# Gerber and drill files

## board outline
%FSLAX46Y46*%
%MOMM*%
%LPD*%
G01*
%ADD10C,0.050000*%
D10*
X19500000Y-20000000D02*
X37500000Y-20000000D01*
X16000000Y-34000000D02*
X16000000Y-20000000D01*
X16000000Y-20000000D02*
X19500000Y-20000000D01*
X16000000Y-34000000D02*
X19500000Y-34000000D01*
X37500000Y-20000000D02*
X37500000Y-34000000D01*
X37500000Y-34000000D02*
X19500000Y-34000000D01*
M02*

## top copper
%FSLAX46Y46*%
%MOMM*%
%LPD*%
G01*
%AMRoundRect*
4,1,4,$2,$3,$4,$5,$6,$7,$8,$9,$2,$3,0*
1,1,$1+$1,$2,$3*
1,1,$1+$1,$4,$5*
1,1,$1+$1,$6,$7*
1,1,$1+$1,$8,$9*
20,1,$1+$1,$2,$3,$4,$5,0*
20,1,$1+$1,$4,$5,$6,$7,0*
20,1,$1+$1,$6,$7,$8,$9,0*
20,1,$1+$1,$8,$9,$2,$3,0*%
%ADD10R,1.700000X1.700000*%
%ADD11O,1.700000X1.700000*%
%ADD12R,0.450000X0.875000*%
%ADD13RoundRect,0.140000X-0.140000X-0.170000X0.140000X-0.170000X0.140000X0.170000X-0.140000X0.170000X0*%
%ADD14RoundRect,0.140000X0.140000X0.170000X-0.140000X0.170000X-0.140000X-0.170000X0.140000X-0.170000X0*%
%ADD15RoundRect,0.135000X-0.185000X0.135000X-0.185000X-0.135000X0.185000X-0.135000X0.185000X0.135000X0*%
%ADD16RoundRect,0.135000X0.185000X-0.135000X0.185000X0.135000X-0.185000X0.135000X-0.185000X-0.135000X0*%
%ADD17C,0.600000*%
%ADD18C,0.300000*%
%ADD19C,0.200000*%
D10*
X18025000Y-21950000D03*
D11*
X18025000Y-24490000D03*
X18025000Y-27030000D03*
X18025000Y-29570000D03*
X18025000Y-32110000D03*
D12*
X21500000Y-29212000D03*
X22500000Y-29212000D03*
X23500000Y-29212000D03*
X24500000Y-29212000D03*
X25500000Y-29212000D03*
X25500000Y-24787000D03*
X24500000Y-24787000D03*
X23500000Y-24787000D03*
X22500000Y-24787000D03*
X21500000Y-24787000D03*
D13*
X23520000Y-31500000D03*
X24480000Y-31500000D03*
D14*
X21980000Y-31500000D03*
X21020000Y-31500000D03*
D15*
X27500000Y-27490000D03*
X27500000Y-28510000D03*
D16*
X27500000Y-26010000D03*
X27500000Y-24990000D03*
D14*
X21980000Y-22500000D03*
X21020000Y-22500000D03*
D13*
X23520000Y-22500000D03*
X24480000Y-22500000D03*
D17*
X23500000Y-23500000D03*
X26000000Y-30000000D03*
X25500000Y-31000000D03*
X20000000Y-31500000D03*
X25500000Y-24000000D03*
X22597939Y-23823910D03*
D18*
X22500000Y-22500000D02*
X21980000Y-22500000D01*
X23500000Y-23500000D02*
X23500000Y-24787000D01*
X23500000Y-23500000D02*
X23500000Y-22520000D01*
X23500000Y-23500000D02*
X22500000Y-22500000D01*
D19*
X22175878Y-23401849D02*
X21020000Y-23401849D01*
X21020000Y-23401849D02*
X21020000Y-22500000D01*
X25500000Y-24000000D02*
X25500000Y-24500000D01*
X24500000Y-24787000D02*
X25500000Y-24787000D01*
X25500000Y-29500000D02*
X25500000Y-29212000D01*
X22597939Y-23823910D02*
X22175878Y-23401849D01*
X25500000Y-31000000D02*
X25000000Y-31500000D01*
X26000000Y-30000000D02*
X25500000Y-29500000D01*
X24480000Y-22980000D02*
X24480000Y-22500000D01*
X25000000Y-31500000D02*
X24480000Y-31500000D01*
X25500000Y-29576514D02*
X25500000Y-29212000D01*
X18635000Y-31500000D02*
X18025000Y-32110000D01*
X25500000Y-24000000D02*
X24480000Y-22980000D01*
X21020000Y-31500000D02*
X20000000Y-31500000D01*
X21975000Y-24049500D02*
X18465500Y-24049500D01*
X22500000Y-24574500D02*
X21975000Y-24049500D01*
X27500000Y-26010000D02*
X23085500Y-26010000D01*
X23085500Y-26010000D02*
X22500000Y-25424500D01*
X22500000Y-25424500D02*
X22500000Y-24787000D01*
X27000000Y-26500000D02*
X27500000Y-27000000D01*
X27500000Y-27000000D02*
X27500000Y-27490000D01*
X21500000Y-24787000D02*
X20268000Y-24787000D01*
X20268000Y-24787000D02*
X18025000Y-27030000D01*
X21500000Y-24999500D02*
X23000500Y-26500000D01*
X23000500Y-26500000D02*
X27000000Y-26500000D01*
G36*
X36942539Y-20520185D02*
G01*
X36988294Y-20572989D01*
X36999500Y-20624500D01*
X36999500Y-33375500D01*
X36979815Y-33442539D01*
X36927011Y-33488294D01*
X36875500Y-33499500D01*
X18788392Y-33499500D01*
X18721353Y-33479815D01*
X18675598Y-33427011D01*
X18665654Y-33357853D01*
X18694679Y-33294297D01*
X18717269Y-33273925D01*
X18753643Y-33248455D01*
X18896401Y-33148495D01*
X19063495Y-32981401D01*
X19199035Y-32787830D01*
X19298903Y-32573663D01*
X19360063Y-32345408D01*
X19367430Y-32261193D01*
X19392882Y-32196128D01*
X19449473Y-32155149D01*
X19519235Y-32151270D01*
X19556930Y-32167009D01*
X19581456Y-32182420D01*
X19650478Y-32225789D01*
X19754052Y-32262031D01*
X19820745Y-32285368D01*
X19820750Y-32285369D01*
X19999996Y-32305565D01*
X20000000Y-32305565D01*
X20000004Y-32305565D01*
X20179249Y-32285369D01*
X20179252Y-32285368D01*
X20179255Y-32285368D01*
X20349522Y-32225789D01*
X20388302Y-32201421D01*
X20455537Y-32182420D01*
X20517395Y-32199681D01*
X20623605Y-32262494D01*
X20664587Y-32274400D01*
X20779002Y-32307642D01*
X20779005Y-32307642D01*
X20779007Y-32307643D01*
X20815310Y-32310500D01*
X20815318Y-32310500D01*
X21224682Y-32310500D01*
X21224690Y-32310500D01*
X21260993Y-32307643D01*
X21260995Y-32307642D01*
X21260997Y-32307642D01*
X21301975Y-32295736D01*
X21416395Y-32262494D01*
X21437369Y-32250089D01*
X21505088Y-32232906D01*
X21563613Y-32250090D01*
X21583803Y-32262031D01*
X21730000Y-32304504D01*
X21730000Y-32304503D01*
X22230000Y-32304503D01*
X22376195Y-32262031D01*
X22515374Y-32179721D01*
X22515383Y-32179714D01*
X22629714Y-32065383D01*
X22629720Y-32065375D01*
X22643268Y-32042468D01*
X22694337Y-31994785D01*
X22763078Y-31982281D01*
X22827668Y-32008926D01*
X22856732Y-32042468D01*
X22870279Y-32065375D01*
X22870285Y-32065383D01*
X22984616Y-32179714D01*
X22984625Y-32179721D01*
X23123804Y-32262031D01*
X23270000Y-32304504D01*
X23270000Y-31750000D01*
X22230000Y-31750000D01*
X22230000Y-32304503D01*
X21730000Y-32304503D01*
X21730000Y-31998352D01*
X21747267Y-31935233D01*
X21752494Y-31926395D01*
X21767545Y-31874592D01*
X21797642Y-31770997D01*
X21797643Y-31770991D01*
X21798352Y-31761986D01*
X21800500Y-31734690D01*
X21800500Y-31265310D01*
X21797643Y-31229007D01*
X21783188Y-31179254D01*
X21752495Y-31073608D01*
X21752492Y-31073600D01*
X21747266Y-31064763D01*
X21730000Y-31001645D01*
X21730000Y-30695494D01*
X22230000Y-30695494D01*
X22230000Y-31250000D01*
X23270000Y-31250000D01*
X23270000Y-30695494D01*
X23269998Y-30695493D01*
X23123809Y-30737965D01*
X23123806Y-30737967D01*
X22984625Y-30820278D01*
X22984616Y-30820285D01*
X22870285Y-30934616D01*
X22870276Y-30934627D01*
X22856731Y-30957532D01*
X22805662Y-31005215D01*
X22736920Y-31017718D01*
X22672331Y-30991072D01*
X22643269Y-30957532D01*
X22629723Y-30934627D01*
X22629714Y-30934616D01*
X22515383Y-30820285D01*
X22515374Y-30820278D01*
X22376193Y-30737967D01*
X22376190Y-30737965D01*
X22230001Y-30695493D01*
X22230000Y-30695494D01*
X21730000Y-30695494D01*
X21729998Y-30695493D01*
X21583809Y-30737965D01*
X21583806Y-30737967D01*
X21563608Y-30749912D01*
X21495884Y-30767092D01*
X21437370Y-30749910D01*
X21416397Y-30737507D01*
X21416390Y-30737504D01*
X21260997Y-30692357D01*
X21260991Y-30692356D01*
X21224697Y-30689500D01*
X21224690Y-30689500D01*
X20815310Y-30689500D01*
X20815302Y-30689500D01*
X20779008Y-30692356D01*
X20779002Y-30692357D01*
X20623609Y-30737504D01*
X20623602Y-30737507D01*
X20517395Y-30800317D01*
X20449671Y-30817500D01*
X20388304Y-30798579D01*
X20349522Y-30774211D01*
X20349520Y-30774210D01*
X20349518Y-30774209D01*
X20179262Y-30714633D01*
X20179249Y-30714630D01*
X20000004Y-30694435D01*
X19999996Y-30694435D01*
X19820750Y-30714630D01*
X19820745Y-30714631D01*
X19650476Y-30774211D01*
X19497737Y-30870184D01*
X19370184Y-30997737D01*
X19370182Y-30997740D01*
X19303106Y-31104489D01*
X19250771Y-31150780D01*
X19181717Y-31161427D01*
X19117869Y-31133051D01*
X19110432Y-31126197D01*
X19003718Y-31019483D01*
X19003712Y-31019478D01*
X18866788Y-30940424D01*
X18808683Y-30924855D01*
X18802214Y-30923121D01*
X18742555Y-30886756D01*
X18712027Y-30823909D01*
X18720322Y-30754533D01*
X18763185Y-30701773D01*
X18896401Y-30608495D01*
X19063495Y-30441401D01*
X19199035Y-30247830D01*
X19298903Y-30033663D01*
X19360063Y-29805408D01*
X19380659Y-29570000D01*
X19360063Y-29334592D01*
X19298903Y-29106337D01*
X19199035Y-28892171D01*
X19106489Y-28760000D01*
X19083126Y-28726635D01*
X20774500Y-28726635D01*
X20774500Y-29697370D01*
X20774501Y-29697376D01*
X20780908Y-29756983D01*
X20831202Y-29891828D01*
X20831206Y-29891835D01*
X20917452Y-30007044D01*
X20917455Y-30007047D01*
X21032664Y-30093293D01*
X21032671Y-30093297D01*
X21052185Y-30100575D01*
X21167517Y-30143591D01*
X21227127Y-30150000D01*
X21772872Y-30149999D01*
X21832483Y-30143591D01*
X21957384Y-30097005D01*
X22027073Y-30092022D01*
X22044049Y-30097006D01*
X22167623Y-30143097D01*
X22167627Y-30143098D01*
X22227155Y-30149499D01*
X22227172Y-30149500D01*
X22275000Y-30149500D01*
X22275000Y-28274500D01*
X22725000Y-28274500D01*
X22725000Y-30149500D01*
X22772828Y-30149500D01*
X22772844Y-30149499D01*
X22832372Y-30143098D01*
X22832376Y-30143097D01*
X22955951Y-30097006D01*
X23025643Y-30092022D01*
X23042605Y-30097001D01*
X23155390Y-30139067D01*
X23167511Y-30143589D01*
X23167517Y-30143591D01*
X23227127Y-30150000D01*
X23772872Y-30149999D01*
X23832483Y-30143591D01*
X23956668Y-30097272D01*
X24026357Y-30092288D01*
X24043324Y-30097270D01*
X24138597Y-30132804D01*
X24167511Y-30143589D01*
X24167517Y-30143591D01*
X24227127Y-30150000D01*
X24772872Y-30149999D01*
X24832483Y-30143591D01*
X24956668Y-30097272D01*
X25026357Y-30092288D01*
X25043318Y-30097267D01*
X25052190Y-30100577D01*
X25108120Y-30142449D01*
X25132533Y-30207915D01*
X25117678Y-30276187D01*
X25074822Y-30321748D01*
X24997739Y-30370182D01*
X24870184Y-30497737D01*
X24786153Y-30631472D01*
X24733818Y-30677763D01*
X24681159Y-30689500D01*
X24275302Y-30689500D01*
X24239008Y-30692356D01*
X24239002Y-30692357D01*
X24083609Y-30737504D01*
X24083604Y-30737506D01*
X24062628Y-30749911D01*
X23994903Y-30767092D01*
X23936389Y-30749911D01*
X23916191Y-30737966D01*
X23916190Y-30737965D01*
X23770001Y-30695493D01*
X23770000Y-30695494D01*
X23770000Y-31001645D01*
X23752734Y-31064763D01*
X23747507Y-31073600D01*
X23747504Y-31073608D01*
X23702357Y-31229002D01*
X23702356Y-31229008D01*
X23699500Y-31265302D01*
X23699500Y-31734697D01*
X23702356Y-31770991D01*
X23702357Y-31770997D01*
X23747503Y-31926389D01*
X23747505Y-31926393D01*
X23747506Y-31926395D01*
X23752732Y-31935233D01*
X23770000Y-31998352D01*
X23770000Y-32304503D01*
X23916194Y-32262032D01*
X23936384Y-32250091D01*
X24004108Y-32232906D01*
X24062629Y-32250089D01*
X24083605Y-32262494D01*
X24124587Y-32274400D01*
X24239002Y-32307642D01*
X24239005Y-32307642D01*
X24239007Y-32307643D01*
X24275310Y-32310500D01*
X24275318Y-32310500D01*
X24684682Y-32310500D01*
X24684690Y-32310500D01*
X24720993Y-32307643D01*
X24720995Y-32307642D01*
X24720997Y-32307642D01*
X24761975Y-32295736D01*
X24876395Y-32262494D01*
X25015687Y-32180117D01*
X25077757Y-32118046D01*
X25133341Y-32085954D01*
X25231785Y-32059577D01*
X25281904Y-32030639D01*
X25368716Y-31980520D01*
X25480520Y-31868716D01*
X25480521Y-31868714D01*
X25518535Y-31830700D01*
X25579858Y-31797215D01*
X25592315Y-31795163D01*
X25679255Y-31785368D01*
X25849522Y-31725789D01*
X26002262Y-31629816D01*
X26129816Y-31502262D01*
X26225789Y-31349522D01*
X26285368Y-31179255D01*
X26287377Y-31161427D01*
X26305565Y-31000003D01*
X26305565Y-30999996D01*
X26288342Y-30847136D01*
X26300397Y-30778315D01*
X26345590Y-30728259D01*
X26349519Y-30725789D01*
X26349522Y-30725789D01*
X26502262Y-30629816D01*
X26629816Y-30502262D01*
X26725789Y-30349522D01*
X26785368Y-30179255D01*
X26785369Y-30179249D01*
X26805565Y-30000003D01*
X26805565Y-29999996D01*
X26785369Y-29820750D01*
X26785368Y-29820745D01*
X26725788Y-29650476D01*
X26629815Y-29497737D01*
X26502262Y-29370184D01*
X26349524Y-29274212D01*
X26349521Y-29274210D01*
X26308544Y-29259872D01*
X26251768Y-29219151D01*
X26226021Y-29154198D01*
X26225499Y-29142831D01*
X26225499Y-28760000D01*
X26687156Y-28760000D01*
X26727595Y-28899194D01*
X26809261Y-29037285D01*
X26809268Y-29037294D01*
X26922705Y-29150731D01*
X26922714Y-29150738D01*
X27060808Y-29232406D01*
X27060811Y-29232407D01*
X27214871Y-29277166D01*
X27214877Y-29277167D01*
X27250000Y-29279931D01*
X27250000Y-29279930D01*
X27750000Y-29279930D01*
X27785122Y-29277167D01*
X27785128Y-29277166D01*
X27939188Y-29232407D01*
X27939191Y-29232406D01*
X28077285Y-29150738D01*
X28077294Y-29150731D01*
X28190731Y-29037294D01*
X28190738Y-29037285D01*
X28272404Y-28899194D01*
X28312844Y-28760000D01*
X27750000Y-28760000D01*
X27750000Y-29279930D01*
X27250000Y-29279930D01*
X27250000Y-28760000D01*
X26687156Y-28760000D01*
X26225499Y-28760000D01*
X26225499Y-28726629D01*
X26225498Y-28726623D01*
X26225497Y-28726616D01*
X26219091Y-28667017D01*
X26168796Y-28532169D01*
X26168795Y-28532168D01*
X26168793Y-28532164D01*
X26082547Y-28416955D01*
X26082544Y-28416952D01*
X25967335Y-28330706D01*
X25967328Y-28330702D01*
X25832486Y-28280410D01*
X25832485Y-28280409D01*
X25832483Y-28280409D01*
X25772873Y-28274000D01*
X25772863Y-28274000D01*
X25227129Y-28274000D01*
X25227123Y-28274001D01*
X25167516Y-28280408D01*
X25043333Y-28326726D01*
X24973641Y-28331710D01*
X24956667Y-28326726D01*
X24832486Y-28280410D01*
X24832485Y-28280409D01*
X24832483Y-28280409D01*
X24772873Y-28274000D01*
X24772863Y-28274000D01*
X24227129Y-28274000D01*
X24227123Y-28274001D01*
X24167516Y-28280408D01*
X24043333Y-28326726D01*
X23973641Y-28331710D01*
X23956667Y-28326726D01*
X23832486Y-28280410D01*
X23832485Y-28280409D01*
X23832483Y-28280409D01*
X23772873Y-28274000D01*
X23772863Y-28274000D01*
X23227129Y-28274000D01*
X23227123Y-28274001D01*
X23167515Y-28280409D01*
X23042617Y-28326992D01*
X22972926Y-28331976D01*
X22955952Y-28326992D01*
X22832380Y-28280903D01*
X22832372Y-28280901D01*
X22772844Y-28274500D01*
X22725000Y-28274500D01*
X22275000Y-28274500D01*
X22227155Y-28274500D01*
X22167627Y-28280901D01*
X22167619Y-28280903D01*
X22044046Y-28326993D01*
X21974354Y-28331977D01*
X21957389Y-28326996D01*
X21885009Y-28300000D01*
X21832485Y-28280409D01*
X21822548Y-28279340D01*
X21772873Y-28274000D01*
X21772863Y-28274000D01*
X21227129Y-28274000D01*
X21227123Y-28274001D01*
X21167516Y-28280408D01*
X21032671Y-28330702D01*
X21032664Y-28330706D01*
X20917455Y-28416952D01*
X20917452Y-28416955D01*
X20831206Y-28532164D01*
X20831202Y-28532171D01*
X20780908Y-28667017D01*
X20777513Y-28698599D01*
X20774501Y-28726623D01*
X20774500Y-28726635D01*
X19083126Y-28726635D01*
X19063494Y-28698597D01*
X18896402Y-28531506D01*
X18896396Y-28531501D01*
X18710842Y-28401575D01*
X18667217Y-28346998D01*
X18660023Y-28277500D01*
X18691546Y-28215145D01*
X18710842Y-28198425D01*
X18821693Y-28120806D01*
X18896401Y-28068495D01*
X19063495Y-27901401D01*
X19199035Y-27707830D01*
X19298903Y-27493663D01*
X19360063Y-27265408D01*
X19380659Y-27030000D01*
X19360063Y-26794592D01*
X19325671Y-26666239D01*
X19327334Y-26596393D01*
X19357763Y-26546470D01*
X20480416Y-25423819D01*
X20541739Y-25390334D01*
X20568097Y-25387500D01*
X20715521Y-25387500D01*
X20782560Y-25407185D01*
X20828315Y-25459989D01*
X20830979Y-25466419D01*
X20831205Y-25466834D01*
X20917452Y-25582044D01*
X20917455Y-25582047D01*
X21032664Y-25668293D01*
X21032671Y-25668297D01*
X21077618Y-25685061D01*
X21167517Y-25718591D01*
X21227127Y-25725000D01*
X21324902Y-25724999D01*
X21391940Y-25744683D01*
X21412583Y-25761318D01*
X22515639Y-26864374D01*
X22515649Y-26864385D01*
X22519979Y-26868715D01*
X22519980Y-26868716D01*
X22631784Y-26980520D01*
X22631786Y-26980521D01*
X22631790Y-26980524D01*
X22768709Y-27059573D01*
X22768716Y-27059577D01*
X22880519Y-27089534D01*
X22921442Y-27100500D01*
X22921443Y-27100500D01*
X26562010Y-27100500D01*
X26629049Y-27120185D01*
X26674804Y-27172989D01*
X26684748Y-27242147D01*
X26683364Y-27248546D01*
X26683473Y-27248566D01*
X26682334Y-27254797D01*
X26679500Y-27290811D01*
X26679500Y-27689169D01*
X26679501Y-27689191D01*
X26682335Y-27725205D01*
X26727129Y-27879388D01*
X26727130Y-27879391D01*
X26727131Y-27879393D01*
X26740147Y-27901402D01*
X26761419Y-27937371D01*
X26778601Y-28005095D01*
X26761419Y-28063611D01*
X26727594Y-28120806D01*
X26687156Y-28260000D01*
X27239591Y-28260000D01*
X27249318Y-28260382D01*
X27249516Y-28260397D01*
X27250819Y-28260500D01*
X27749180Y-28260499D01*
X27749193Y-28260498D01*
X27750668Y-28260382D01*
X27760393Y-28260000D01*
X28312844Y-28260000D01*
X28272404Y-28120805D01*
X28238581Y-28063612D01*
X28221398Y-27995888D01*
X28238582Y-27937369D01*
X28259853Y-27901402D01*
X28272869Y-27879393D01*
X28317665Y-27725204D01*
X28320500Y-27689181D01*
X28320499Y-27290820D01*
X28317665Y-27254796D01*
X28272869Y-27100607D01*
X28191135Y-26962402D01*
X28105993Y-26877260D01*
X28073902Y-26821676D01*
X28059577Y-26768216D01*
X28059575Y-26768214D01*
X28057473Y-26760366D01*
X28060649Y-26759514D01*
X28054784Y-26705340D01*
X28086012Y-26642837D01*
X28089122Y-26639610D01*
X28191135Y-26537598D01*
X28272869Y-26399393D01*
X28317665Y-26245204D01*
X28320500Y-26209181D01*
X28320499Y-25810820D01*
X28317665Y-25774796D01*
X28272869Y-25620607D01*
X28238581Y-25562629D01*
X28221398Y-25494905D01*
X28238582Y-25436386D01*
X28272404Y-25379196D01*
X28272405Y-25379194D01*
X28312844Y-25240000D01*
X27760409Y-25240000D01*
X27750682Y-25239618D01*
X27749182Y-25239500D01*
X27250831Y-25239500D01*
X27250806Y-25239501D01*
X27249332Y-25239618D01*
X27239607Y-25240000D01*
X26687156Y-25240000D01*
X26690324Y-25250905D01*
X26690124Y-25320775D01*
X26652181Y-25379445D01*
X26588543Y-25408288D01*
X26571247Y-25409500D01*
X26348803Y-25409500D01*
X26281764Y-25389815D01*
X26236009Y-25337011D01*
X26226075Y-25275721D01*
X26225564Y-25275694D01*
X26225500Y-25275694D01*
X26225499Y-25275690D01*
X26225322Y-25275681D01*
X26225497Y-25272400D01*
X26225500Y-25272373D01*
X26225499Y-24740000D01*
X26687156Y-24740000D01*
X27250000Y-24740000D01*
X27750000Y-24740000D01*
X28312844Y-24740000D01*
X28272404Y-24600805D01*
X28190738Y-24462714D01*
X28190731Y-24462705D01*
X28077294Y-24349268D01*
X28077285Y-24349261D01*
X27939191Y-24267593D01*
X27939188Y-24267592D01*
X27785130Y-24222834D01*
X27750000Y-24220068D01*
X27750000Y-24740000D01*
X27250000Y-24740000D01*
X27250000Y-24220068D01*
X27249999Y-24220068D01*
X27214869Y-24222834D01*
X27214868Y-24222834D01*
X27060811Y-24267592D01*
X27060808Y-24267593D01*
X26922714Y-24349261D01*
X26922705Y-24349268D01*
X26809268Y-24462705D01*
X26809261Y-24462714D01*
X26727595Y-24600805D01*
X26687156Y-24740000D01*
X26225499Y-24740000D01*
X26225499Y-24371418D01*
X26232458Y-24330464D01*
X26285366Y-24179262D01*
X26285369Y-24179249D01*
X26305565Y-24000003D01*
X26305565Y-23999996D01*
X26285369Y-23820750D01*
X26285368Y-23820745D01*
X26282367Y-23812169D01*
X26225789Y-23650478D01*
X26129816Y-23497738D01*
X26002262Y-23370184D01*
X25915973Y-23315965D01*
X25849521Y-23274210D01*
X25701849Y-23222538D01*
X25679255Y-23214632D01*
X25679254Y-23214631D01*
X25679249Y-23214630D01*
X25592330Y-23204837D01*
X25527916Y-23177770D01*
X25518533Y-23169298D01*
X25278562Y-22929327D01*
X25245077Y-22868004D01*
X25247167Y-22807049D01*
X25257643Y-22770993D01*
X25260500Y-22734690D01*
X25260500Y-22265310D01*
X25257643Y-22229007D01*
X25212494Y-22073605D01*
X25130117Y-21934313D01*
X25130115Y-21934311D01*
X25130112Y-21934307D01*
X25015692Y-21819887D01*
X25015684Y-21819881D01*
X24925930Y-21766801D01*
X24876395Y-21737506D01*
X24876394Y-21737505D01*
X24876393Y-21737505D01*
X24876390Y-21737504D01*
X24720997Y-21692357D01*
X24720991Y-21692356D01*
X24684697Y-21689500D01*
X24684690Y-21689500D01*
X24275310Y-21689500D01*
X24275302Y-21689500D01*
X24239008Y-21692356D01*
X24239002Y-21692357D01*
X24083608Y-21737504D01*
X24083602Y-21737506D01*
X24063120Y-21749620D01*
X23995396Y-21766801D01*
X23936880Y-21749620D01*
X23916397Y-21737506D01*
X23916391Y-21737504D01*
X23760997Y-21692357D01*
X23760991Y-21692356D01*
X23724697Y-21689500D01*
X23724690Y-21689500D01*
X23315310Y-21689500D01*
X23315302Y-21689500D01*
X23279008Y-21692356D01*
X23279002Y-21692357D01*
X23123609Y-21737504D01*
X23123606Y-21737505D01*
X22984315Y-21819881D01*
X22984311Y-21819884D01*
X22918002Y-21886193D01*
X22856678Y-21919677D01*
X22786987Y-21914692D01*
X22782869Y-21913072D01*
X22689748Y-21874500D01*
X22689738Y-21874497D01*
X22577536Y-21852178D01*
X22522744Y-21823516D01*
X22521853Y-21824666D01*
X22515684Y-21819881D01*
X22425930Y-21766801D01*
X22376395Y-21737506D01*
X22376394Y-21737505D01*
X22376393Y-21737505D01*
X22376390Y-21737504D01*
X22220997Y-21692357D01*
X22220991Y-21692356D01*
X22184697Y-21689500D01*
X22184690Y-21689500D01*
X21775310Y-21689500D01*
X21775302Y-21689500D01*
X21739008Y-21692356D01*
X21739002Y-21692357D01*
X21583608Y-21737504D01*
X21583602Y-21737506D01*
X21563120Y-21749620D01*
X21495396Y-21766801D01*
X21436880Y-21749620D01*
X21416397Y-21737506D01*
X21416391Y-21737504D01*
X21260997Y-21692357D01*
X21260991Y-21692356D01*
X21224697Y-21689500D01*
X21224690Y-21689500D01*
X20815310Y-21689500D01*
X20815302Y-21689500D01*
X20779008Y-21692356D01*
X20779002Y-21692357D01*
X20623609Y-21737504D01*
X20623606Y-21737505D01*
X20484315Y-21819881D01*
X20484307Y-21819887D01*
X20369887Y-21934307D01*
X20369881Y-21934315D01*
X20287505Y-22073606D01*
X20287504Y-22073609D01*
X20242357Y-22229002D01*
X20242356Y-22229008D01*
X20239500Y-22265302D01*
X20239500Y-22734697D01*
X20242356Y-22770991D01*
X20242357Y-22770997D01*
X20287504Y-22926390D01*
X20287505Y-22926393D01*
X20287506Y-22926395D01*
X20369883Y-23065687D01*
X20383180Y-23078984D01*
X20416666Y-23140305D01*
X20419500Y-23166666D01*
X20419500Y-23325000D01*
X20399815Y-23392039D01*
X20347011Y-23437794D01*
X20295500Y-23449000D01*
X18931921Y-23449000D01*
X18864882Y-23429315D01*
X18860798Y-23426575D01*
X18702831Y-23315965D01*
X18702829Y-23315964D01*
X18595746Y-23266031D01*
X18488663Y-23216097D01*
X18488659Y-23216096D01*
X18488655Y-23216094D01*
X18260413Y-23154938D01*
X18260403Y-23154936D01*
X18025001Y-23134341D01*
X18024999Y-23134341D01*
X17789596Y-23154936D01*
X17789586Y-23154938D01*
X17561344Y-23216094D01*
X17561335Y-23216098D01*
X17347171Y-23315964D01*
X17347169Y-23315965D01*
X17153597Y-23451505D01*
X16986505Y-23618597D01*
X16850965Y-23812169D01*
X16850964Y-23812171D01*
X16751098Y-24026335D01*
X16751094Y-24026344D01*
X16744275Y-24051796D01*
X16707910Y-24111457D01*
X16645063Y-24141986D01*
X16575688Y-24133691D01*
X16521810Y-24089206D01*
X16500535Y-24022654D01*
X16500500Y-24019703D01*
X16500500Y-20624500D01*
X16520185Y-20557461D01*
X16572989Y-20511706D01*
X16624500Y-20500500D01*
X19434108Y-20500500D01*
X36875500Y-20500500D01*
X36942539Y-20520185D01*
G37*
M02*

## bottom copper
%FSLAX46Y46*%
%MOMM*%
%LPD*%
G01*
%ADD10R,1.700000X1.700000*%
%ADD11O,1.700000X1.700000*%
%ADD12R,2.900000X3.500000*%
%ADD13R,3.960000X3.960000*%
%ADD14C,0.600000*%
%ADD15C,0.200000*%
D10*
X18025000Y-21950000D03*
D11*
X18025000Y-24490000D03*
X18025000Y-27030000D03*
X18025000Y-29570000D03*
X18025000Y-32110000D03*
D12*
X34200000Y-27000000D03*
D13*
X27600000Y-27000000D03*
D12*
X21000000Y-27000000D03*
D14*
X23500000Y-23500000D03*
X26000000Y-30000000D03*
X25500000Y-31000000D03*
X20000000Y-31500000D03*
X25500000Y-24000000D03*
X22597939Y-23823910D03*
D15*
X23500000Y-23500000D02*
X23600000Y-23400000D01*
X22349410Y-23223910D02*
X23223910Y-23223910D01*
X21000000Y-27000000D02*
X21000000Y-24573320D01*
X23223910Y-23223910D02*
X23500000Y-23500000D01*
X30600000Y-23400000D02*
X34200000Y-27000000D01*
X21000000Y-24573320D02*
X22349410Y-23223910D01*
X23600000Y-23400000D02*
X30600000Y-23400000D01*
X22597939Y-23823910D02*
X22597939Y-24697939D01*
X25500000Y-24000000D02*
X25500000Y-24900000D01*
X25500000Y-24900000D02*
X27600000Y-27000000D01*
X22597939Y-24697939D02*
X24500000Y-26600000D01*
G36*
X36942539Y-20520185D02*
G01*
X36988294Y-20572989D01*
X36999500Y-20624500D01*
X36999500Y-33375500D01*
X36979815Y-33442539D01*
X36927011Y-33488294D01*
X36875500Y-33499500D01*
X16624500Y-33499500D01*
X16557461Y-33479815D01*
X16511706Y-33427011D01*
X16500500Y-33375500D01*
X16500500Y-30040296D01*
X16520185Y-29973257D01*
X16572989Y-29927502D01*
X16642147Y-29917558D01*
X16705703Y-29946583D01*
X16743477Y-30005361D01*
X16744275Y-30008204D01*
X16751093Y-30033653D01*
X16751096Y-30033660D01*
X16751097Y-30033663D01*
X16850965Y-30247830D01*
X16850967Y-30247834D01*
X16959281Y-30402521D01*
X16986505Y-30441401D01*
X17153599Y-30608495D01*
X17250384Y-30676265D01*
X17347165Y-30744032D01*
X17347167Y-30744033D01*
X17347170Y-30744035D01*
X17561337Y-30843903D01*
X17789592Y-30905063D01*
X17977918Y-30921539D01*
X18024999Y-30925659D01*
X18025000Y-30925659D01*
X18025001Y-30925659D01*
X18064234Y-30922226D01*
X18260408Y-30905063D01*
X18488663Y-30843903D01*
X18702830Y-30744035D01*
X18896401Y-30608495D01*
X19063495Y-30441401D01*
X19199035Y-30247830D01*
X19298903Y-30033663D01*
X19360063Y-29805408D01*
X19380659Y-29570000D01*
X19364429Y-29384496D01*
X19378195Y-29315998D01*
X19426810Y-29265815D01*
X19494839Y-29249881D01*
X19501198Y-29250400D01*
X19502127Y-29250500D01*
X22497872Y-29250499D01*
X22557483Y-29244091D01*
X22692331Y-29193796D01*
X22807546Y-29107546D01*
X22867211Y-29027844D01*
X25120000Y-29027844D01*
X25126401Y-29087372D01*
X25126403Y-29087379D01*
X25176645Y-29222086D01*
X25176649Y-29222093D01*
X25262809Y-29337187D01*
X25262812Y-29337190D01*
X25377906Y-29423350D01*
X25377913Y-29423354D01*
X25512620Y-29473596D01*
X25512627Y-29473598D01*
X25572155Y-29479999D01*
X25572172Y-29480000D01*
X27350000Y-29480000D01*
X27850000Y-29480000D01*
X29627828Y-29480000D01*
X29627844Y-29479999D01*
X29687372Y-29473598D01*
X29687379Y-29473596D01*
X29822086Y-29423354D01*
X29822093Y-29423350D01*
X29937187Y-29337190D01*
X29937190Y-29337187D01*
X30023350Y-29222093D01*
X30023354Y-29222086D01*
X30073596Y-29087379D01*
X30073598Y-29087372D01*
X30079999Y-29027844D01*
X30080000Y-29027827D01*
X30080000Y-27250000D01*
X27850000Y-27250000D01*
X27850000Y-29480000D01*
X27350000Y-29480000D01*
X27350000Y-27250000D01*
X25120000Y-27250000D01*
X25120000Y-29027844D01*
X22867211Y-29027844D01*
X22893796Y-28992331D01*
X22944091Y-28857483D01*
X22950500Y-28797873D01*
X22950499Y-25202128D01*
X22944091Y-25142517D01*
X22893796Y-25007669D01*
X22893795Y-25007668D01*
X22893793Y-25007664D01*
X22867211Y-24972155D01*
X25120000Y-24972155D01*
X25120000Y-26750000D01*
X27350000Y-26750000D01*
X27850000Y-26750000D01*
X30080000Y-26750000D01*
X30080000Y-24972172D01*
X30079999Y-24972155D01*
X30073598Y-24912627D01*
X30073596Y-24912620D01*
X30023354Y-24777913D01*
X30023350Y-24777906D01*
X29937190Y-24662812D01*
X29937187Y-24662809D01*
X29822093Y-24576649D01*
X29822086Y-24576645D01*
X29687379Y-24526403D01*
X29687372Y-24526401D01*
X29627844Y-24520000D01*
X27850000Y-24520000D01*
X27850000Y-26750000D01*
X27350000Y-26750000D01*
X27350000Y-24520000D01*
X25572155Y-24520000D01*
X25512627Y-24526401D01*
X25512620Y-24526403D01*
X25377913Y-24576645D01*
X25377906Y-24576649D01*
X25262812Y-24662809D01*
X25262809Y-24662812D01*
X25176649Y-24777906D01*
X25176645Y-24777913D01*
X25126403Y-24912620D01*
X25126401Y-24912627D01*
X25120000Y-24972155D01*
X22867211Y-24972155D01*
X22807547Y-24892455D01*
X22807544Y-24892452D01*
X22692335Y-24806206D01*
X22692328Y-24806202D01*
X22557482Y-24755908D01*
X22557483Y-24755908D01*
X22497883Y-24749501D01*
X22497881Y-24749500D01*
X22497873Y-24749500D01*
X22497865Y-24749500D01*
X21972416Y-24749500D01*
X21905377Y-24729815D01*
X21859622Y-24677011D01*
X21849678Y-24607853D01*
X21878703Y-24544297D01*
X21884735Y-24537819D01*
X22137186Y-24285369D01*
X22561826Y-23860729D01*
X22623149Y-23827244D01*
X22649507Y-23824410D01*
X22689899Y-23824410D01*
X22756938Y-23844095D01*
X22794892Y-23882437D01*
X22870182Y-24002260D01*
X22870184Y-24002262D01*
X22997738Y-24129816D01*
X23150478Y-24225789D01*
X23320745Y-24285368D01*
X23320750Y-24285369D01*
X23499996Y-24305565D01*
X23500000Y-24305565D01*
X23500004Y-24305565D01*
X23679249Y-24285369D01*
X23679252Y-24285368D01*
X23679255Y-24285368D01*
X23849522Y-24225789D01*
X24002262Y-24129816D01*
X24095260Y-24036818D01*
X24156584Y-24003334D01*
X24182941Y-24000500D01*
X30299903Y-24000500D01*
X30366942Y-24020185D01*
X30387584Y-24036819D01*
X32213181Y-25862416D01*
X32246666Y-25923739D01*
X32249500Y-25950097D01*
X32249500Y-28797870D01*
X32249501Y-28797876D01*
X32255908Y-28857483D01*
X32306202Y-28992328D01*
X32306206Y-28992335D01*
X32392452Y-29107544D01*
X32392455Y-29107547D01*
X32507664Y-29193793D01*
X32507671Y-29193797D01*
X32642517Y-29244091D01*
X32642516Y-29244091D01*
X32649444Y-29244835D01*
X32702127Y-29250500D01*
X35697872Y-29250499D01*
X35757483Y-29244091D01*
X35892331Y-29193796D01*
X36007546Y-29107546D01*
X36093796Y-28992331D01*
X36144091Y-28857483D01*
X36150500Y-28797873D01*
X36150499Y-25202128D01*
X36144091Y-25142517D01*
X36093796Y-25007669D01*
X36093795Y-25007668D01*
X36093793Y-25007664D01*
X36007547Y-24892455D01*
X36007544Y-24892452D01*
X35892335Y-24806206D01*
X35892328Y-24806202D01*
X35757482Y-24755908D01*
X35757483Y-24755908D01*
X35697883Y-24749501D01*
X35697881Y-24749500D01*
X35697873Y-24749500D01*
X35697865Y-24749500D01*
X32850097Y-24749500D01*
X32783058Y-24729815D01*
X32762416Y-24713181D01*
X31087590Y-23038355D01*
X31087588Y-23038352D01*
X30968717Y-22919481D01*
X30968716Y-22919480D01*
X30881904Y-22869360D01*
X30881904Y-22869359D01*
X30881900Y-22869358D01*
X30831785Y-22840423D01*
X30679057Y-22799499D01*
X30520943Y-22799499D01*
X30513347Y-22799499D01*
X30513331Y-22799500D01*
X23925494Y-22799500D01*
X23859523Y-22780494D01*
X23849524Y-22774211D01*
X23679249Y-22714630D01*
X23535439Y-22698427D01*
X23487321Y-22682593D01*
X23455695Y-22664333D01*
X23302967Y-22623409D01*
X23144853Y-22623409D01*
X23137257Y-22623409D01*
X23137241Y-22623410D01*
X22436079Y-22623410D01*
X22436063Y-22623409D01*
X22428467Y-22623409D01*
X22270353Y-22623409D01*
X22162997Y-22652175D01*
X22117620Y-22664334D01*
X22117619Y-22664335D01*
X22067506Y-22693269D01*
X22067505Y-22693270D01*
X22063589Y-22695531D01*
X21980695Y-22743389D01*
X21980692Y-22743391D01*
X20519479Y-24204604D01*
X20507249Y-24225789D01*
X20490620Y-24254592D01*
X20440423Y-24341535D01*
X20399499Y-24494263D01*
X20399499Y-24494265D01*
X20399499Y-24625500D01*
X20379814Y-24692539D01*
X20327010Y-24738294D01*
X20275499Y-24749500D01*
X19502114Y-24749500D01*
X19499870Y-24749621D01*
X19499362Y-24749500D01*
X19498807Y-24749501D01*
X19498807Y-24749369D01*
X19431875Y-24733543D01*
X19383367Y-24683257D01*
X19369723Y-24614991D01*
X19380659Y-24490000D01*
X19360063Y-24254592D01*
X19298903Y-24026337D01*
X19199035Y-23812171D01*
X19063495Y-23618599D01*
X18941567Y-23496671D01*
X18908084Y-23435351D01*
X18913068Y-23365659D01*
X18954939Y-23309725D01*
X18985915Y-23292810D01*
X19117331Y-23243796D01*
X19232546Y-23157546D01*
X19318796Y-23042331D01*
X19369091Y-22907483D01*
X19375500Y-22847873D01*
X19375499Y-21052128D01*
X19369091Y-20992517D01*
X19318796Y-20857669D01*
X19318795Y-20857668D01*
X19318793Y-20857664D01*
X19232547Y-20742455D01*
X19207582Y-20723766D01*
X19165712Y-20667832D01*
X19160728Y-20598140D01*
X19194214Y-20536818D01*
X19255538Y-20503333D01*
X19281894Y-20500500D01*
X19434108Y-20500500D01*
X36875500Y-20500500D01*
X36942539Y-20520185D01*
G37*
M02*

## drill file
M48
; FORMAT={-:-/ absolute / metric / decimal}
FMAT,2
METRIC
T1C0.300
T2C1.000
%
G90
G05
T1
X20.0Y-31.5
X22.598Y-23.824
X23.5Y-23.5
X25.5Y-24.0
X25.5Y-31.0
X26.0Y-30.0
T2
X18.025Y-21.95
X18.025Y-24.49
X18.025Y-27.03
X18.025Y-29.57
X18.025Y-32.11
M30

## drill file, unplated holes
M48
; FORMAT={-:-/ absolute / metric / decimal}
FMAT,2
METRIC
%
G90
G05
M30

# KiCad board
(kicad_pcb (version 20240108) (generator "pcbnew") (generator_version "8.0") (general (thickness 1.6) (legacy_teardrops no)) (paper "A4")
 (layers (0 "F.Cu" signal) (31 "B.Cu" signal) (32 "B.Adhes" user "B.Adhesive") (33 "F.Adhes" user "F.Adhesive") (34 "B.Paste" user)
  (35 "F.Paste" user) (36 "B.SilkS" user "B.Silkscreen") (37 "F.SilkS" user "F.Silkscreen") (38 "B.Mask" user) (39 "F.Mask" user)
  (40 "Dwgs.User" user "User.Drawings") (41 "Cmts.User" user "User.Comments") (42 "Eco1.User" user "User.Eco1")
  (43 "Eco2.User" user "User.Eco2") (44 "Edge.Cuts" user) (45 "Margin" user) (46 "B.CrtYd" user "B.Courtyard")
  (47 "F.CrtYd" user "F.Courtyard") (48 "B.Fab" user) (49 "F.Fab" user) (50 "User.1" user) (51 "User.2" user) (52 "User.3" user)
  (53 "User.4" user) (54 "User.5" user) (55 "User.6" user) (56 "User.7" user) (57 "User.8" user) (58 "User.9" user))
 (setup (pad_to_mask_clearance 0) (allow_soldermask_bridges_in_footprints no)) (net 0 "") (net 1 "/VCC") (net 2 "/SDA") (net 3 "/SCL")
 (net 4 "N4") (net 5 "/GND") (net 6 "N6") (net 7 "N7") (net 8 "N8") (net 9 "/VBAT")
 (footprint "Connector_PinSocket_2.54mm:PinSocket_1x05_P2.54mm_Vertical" (layer "F.Cu") (at 18.025 21.95)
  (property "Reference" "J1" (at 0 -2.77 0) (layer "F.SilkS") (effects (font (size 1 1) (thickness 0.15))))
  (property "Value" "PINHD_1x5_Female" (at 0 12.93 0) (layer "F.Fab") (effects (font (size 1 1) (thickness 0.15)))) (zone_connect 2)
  (pad "1" thru_hole rect (at 0 0) (size 1.7 1.7) (drill 1) (layers "*.Cu" "*.Mask") (remove_unused_layers no) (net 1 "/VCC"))
  (pad "2" thru_hole oval (at 0 2.54) (size 1.7 1.7) (drill 1) (layers "*.Cu" "*.Mask") (remove_unused_layers no) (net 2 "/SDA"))
  (pad "3" thru_hole oval (at 0 5.08) (size 1.7 1.7) (drill 1) (layers "*.Cu" "*.Mask") (remove_unused_layers no) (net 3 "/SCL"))
  (pad "4" thru_hole oval (at 0 7.62) (size 1.7 1.7) (drill 1) (layers "*.Cu" "*.Mask") (remove_unused_layers no) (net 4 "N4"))
  (pad "5" thru_hole oval (at 0 10.16) (size 1.7 1.7) (drill 1) (layers "*.Cu" "*.Mask") (remove_unused_layers no) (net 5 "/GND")))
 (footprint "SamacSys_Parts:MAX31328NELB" (layer "F.Cu") (at 23.5 27)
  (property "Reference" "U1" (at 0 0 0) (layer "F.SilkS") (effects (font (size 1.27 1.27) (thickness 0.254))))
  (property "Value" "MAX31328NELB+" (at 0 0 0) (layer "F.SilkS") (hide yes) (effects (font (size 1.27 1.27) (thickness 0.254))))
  (pad "1" smd rect (at -2 2.212) (size 0.45 0.875) (layers "F.Cu" "F.Paste" "F.Mask") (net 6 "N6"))
  (pad "2" smd rect (at -1 2.212) (size 0.45 0.875) (layers "F.Cu" "F.Paste" "F.Mask") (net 1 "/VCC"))
  (pad "3" smd rect (at 0 2.212) (size 0.45 0.875) (layers "F.Cu" "F.Paste" "F.Mask") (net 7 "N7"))
  (pad "4" smd rect (at 1 2.212) (size 0.45 0.875) (layers "F.Cu" "F.Paste" "F.Mask") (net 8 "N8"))
  (pad "5" smd rect (at 2 2.212) (size 0.45 0.875) (layers "F.Cu" "F.Paste" "F.Mask") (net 5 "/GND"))
  (pad "6" smd rect (at 2 -2.213) (size 0.45 0.875) (layers "F.Cu" "F.Paste" "F.Mask") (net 5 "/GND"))
  (pad "7" smd rect (at 1 -2.213) (size 0.45 0.875) (layers "F.Cu" "F.Paste" "F.Mask") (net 5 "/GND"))
  (pad "8" smd rect (at 0 -2.213) (size 0.45 0.875) (layers "F.Cu" "F.Paste" "F.Mask") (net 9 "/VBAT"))
  (pad "9" smd rect (at -1 -2.213) (size 0.45 0.875) (layers "F.Cu" "F.Paste" "F.Mask") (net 2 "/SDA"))
  (pad "10" smd rect (at -2 -2.213) (size 0.45 0.875) (layers "F.Cu" "F.Paste" "F.Mask") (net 3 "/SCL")))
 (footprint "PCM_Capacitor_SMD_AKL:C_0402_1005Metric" (layer "F.Cu") (at 24 31.5)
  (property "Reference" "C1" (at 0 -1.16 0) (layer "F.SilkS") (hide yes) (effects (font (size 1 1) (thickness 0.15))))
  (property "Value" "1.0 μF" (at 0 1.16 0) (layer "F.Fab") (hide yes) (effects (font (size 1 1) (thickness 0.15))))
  (pad "1" smd roundrect (at -0.48 0) (size 0.56 0.62) (layers "F.Cu" "F.Paste" "F.Mask") (roundrect_rratio 0.25) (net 1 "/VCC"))
  (pad "2" smd roundrect (at 0.48 0) (size 0.56 0.62) (layers "F.Cu" "F.Paste" "F.Mask") (roundrect_rratio 0.25) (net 5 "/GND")))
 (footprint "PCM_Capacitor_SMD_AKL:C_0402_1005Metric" (layer "F.Cu") (at 21.5 31.5 180)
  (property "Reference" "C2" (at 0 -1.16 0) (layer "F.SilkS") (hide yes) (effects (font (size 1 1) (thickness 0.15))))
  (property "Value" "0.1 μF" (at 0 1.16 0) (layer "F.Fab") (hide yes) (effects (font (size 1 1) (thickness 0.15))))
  (pad "1" smd roundrect (at -0.48 0 180) (size 0.56 0.62) (layers "F.Cu" "F.Paste" "F.Mask") (roundrect_rratio 0.25) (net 1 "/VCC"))
  (pad "2" smd roundrect (at 0.48 0 180) (size 0.56 0.62) (layers "F.Cu" "F.Paste" "F.Mask") (roundrect_rratio 0.25) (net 5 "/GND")))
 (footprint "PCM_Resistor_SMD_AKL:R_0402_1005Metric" (layer "F.Cu") (at 27.5 28 -90)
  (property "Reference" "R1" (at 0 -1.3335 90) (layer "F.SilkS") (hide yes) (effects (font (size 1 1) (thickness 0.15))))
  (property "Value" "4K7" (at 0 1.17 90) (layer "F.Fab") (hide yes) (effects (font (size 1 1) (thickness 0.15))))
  (pad "1" smd roundrect (at -0.51 0 270) (size 0.54 0.64) (layers "F.Cu" "F.Paste" "F.Mask") (roundrect_rratio 0.25) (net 3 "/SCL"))
  (pad "2" smd roundrect (at 0.51 0 270) (size 0.54 0.64) (layers "F.Cu" "F.Paste" "F.Mask") (roundrect_rratio 0.25) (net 1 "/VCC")))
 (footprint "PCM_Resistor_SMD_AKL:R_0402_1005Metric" (layer "F.Cu") (at 27.5 25.5 90)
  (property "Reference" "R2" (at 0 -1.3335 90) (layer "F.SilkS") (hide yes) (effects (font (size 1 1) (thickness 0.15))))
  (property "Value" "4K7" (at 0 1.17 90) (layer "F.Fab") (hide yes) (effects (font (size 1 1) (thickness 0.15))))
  (pad "1" smd roundrect (at -0.51 0 90) (size 0.54 0.64) (layers "F.Cu" "F.Paste" "F.Mask") (roundrect_rratio 0.25) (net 2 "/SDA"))
  (pad "2" smd roundrect (at 0.51 0 90) (size 0.54 0.64) (layers "F.Cu" "F.Paste" "F.Mask") (roundrect_rratio 0.25) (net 1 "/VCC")))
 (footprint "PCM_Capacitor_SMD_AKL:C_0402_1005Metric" (layer "F.Cu") (at 21.5 22.5 180)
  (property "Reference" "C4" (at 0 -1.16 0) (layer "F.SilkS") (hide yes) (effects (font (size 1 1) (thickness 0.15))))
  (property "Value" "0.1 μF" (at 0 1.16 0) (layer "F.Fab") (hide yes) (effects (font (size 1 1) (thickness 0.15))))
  (pad "1" smd roundrect (at -0.48 0 180) (size 0.56 0.62) (layers "F.Cu" "F.Paste" "F.Mask") (roundrect_rratio 0.25) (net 9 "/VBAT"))
  (pad "2" smd roundrect (at 0.48 0 180) (size 0.56 0.62) (layers "F.Cu" "F.Paste" "F.Mask") (roundrect_rratio 0.25) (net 5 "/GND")))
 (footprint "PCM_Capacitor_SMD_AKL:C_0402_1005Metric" (layer "F.Cu") (at 24 22.5)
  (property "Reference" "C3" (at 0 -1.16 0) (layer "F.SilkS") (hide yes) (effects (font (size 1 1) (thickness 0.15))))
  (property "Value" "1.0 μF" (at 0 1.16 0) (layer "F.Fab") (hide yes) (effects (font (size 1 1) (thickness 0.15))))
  (pad "1" smd roundrect (at -0.48 0) (size 0.56 0.62) (layers "F.Cu" "F.Paste" "F.Mask") (roundrect_rratio 0.25) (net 9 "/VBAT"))
  (pad "2" smd roundrect (at 0.48 0) (size 0.56 0.62) (layers "F.Cu" "F.Paste" "F.Mask") (roundrect_rratio 0.25) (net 5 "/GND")))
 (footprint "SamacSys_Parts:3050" (layer "B.Cu") (at 27.6 27 180)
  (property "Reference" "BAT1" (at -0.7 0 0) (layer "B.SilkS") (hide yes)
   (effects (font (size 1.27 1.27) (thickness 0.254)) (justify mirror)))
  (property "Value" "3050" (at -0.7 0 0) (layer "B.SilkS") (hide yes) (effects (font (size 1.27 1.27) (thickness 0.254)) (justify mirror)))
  (pad "1" smd rect (at -6.6 0 180) (size 2.9 3.5) (layers "B.Cu" "B.Paste" "B.Mask") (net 9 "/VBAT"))
  (pad "2" smd rect (at 0 0 90) (size 3.96 3.96) (layers "B.Cu" "B.Paste" "B.Mask") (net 5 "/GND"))
  (pad "3" smd rect (at 6.6 0 180) (size 2.9 3.5) (layers "B.Cu" "B.Paste" "B.Mask") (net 9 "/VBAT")))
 (gr_line (start 19.5 20) (end 37.5 20) (stroke (width 0.05) (type default)) (layer "Edge.Cuts"))
 (gr_line (start 16 34) (end 16 20) (stroke (width 0.05) (type default)) (layer "Edge.Cuts"))
 (gr_line (start 16 20) (end 19.5 20) (stroke (width 0.05) (type default)) (layer "Edge.Cuts"))
 (gr_line (start 16 34) (end 19.5 34) (stroke (width 0.05) (type default)) (layer "Edge.Cuts"))
 (gr_line (start 37.5 20) (end 37.5 34) (stroke (width 0.05) (type default)) (layer "Edge.Cuts"))
 (gr_line (start 37.5 34) (end 19.5 34) (stroke (width 0.05) (type default)) (layer "Edge.Cuts"))
 (segment (start 22.5 22.5) (end 21.98 22.5) (width 0.3) (layer "F.Cu") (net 9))
 (segment (start 23.5 23.5) (end 23.5 24.787) (width 0.3) (layer "F.Cu") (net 9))
 (segment (start 23.5 23.5) (end 23.5 22.52) (width 0.3) (layer "F.Cu") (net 9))
 (segment (start 23.5 23.5) (end 22.5 22.5) (width 0.3) (layer "F.Cu") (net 9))
 (via (at 23.5 23.5) (size 0.6) (drill 0.3) (layers "F.Cu" "B.Cu") (remove_unused_layers yes) (keep_end_layers yes) (free yes)
  (zone_layer_connections) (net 9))
 (segment (start 23.5 23.5) (end 23.6 23.4) (width 0.2) (layer "B.Cu") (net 9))
 (segment (start 22.34941 23.22391) (end 23.22391 23.22391) (width 0.2) (layer "B.Cu") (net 9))
 (segment (start 21 27) (end 21 24.57332) (width 0.2) (layer "B.Cu") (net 9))
 (segment (start 23.22391 23.22391) (end 23.5 23.5) (width 0.2) (layer "B.Cu") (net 9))
 (segment (start 30.6 23.4) (end 34.2 27) (width 0.2) (layer "B.Cu") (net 9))
 (segment (start 21 24.57332) (end 22.34941 23.22391) (width 0.2) (layer "B.Cu") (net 9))
 (segment (start 23.6 23.4) (end 30.6 23.4) (width 0.2) (layer "B.Cu") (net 9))
 (segment (start 22.175878 23.401849) (end 21.02 23.401849) (width 0.2) (layer "F.Cu") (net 5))
 (segment (start 21.02 23.401849) (end 21.02 22.5) (width 0.2) (layer "F.Cu") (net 5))
 (segment (start 25.5 24) (end 25.5 24.5) (width 0.2) (layer "F.Cu") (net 5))
 (segment (start 24.5 24.787) (end 25.5 24.787) (width 0.2) (layer "F.Cu") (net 5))
 (segment (start 25.5 29.5) (end 25.5 29.212) (width 0.2) (layer "F.Cu") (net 5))
 (segment (start 22.597939 23.82391) (end 22.175878 23.401849) (width 0.2) (layer "F.Cu") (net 5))
 (segment (start 25.5 31) (end 25 31.5) (width 0.2) (layer "F.Cu") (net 5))
 (segment (start 26 30) (end 25.5 29.5) (width 0.2) (layer "F.Cu") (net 5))
 (segment (start 24.48 22.98) (end 24.48 22.5) (width 0.2) (layer "F.Cu") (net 5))
 (segment (start 25 31.5) (end 24.48 31.5) (width 0.2) (layer "F.Cu") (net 5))
 (segment (start 25.5 29.576514) (end 25.5 29.212) (width 0.2) (layer "F.Cu") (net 5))
 (segment (start 18.635 31.5) (end 18.025 32.11) (width 0.2) (layer "F.Cu") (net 5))
 (segment (start 25.5 24) (end 24.48 22.98) (width 0.2) (layer "F.Cu") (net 5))
 (segment (start 21.02 31.5) (end 20 31.5) (width 0.2) (layer "F.Cu") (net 5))
 (via (at 26 30) (size 0.6) (drill 0.3) (layers "F.Cu" "B.Cu") (free yes) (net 5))
 (via (at 25.5 31) (size 0.6) (drill 0.3) (layers "F.Cu" "B.Cu") (remove_unused_layers yes) (keep_end_layers yes) (free yes)
  (zone_layer_connections) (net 5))
 (via (at 20 31.5) (size 0.6) (drill 0.3) (layers "F.Cu" "B.Cu") (free yes) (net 5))
 (via (at 25.5 24) (size 0.6) (drill 0.3) (layers "F.Cu" "B.Cu") (remove_unused_layers yes) (keep_end_layers yes) (free yes)
  (zone_layer_connections) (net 5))
 (via (at 22.597939 23.82391) (size 0.6) (drill 0.3) (layers "F.Cu" "B.Cu") (remove_unused_layers yes) (keep_end_layers yes) (free yes)
  (zone_layer_connections) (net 5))
 (segment (start 22.597939 23.82391) (end 22.597939 24.697939) (width 0.2) (layer "B.Cu") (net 5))
 (segment (start 25.5 24) (end 25.5 24.9) (width 0.2) (layer "B.Cu") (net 5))
 (segment (start 25.5 24.9) (end 27.6 27) (width 0.2) (layer "B.Cu") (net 5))
 (segment (start 22.597939 24.697939) (end 24.5 26.6) (width 0.2) (layer "B.Cu") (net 5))
 (segment (start 21.975 24.0495) (end 18.4655 24.0495) (width 0.2) (layer "F.Cu") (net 2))
 (segment (start 22.5 24.5745) (end 21.975 24.0495) (width 0.2) (layer "F.Cu") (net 2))
 (segment (start 27.5 26.01) (end 23.0855 26.01) (width 0.2) (layer "F.Cu") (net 2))
 (segment (start 23.0855 26.01) (end 22.5 25.4245) (width 0.2) (layer "F.Cu") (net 2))
 (segment (start 22.5 25.4245) (end 22.5 24.787) (width 0.2) (layer "F.Cu") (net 2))
 (segment (start 27 26.5) (end 27.5 27) (width 0.2) (layer "F.Cu") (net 3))
 (segment (start 27.5 27) (end 27.5 27.49) (width 0.2) (layer "F.Cu") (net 3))
 (segment (start 21.5 24.787) (end 20.268 24.787) (width 0.2) (layer "F.Cu") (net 3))
 (segment (start 20.268 24.787) (end 18.025 27.03) (width 0.2) (layer "F.Cu") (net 3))
 (segment (start 21.5 24.9995) (end 23.0005 26.5) (width 0.2) (layer "F.Cu") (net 3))
 (segment (start 23.0005 26.5) (end 27 26.5) (width 0.2) (layer "F.Cu") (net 3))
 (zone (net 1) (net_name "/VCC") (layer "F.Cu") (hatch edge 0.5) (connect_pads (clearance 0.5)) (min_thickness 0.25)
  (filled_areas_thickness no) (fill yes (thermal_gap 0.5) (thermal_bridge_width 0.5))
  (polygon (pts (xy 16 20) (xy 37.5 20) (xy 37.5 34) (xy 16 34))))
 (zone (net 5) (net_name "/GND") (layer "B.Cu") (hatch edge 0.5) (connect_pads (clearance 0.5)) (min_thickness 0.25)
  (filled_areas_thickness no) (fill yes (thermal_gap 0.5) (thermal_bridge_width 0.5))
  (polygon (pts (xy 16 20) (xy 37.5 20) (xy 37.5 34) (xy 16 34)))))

